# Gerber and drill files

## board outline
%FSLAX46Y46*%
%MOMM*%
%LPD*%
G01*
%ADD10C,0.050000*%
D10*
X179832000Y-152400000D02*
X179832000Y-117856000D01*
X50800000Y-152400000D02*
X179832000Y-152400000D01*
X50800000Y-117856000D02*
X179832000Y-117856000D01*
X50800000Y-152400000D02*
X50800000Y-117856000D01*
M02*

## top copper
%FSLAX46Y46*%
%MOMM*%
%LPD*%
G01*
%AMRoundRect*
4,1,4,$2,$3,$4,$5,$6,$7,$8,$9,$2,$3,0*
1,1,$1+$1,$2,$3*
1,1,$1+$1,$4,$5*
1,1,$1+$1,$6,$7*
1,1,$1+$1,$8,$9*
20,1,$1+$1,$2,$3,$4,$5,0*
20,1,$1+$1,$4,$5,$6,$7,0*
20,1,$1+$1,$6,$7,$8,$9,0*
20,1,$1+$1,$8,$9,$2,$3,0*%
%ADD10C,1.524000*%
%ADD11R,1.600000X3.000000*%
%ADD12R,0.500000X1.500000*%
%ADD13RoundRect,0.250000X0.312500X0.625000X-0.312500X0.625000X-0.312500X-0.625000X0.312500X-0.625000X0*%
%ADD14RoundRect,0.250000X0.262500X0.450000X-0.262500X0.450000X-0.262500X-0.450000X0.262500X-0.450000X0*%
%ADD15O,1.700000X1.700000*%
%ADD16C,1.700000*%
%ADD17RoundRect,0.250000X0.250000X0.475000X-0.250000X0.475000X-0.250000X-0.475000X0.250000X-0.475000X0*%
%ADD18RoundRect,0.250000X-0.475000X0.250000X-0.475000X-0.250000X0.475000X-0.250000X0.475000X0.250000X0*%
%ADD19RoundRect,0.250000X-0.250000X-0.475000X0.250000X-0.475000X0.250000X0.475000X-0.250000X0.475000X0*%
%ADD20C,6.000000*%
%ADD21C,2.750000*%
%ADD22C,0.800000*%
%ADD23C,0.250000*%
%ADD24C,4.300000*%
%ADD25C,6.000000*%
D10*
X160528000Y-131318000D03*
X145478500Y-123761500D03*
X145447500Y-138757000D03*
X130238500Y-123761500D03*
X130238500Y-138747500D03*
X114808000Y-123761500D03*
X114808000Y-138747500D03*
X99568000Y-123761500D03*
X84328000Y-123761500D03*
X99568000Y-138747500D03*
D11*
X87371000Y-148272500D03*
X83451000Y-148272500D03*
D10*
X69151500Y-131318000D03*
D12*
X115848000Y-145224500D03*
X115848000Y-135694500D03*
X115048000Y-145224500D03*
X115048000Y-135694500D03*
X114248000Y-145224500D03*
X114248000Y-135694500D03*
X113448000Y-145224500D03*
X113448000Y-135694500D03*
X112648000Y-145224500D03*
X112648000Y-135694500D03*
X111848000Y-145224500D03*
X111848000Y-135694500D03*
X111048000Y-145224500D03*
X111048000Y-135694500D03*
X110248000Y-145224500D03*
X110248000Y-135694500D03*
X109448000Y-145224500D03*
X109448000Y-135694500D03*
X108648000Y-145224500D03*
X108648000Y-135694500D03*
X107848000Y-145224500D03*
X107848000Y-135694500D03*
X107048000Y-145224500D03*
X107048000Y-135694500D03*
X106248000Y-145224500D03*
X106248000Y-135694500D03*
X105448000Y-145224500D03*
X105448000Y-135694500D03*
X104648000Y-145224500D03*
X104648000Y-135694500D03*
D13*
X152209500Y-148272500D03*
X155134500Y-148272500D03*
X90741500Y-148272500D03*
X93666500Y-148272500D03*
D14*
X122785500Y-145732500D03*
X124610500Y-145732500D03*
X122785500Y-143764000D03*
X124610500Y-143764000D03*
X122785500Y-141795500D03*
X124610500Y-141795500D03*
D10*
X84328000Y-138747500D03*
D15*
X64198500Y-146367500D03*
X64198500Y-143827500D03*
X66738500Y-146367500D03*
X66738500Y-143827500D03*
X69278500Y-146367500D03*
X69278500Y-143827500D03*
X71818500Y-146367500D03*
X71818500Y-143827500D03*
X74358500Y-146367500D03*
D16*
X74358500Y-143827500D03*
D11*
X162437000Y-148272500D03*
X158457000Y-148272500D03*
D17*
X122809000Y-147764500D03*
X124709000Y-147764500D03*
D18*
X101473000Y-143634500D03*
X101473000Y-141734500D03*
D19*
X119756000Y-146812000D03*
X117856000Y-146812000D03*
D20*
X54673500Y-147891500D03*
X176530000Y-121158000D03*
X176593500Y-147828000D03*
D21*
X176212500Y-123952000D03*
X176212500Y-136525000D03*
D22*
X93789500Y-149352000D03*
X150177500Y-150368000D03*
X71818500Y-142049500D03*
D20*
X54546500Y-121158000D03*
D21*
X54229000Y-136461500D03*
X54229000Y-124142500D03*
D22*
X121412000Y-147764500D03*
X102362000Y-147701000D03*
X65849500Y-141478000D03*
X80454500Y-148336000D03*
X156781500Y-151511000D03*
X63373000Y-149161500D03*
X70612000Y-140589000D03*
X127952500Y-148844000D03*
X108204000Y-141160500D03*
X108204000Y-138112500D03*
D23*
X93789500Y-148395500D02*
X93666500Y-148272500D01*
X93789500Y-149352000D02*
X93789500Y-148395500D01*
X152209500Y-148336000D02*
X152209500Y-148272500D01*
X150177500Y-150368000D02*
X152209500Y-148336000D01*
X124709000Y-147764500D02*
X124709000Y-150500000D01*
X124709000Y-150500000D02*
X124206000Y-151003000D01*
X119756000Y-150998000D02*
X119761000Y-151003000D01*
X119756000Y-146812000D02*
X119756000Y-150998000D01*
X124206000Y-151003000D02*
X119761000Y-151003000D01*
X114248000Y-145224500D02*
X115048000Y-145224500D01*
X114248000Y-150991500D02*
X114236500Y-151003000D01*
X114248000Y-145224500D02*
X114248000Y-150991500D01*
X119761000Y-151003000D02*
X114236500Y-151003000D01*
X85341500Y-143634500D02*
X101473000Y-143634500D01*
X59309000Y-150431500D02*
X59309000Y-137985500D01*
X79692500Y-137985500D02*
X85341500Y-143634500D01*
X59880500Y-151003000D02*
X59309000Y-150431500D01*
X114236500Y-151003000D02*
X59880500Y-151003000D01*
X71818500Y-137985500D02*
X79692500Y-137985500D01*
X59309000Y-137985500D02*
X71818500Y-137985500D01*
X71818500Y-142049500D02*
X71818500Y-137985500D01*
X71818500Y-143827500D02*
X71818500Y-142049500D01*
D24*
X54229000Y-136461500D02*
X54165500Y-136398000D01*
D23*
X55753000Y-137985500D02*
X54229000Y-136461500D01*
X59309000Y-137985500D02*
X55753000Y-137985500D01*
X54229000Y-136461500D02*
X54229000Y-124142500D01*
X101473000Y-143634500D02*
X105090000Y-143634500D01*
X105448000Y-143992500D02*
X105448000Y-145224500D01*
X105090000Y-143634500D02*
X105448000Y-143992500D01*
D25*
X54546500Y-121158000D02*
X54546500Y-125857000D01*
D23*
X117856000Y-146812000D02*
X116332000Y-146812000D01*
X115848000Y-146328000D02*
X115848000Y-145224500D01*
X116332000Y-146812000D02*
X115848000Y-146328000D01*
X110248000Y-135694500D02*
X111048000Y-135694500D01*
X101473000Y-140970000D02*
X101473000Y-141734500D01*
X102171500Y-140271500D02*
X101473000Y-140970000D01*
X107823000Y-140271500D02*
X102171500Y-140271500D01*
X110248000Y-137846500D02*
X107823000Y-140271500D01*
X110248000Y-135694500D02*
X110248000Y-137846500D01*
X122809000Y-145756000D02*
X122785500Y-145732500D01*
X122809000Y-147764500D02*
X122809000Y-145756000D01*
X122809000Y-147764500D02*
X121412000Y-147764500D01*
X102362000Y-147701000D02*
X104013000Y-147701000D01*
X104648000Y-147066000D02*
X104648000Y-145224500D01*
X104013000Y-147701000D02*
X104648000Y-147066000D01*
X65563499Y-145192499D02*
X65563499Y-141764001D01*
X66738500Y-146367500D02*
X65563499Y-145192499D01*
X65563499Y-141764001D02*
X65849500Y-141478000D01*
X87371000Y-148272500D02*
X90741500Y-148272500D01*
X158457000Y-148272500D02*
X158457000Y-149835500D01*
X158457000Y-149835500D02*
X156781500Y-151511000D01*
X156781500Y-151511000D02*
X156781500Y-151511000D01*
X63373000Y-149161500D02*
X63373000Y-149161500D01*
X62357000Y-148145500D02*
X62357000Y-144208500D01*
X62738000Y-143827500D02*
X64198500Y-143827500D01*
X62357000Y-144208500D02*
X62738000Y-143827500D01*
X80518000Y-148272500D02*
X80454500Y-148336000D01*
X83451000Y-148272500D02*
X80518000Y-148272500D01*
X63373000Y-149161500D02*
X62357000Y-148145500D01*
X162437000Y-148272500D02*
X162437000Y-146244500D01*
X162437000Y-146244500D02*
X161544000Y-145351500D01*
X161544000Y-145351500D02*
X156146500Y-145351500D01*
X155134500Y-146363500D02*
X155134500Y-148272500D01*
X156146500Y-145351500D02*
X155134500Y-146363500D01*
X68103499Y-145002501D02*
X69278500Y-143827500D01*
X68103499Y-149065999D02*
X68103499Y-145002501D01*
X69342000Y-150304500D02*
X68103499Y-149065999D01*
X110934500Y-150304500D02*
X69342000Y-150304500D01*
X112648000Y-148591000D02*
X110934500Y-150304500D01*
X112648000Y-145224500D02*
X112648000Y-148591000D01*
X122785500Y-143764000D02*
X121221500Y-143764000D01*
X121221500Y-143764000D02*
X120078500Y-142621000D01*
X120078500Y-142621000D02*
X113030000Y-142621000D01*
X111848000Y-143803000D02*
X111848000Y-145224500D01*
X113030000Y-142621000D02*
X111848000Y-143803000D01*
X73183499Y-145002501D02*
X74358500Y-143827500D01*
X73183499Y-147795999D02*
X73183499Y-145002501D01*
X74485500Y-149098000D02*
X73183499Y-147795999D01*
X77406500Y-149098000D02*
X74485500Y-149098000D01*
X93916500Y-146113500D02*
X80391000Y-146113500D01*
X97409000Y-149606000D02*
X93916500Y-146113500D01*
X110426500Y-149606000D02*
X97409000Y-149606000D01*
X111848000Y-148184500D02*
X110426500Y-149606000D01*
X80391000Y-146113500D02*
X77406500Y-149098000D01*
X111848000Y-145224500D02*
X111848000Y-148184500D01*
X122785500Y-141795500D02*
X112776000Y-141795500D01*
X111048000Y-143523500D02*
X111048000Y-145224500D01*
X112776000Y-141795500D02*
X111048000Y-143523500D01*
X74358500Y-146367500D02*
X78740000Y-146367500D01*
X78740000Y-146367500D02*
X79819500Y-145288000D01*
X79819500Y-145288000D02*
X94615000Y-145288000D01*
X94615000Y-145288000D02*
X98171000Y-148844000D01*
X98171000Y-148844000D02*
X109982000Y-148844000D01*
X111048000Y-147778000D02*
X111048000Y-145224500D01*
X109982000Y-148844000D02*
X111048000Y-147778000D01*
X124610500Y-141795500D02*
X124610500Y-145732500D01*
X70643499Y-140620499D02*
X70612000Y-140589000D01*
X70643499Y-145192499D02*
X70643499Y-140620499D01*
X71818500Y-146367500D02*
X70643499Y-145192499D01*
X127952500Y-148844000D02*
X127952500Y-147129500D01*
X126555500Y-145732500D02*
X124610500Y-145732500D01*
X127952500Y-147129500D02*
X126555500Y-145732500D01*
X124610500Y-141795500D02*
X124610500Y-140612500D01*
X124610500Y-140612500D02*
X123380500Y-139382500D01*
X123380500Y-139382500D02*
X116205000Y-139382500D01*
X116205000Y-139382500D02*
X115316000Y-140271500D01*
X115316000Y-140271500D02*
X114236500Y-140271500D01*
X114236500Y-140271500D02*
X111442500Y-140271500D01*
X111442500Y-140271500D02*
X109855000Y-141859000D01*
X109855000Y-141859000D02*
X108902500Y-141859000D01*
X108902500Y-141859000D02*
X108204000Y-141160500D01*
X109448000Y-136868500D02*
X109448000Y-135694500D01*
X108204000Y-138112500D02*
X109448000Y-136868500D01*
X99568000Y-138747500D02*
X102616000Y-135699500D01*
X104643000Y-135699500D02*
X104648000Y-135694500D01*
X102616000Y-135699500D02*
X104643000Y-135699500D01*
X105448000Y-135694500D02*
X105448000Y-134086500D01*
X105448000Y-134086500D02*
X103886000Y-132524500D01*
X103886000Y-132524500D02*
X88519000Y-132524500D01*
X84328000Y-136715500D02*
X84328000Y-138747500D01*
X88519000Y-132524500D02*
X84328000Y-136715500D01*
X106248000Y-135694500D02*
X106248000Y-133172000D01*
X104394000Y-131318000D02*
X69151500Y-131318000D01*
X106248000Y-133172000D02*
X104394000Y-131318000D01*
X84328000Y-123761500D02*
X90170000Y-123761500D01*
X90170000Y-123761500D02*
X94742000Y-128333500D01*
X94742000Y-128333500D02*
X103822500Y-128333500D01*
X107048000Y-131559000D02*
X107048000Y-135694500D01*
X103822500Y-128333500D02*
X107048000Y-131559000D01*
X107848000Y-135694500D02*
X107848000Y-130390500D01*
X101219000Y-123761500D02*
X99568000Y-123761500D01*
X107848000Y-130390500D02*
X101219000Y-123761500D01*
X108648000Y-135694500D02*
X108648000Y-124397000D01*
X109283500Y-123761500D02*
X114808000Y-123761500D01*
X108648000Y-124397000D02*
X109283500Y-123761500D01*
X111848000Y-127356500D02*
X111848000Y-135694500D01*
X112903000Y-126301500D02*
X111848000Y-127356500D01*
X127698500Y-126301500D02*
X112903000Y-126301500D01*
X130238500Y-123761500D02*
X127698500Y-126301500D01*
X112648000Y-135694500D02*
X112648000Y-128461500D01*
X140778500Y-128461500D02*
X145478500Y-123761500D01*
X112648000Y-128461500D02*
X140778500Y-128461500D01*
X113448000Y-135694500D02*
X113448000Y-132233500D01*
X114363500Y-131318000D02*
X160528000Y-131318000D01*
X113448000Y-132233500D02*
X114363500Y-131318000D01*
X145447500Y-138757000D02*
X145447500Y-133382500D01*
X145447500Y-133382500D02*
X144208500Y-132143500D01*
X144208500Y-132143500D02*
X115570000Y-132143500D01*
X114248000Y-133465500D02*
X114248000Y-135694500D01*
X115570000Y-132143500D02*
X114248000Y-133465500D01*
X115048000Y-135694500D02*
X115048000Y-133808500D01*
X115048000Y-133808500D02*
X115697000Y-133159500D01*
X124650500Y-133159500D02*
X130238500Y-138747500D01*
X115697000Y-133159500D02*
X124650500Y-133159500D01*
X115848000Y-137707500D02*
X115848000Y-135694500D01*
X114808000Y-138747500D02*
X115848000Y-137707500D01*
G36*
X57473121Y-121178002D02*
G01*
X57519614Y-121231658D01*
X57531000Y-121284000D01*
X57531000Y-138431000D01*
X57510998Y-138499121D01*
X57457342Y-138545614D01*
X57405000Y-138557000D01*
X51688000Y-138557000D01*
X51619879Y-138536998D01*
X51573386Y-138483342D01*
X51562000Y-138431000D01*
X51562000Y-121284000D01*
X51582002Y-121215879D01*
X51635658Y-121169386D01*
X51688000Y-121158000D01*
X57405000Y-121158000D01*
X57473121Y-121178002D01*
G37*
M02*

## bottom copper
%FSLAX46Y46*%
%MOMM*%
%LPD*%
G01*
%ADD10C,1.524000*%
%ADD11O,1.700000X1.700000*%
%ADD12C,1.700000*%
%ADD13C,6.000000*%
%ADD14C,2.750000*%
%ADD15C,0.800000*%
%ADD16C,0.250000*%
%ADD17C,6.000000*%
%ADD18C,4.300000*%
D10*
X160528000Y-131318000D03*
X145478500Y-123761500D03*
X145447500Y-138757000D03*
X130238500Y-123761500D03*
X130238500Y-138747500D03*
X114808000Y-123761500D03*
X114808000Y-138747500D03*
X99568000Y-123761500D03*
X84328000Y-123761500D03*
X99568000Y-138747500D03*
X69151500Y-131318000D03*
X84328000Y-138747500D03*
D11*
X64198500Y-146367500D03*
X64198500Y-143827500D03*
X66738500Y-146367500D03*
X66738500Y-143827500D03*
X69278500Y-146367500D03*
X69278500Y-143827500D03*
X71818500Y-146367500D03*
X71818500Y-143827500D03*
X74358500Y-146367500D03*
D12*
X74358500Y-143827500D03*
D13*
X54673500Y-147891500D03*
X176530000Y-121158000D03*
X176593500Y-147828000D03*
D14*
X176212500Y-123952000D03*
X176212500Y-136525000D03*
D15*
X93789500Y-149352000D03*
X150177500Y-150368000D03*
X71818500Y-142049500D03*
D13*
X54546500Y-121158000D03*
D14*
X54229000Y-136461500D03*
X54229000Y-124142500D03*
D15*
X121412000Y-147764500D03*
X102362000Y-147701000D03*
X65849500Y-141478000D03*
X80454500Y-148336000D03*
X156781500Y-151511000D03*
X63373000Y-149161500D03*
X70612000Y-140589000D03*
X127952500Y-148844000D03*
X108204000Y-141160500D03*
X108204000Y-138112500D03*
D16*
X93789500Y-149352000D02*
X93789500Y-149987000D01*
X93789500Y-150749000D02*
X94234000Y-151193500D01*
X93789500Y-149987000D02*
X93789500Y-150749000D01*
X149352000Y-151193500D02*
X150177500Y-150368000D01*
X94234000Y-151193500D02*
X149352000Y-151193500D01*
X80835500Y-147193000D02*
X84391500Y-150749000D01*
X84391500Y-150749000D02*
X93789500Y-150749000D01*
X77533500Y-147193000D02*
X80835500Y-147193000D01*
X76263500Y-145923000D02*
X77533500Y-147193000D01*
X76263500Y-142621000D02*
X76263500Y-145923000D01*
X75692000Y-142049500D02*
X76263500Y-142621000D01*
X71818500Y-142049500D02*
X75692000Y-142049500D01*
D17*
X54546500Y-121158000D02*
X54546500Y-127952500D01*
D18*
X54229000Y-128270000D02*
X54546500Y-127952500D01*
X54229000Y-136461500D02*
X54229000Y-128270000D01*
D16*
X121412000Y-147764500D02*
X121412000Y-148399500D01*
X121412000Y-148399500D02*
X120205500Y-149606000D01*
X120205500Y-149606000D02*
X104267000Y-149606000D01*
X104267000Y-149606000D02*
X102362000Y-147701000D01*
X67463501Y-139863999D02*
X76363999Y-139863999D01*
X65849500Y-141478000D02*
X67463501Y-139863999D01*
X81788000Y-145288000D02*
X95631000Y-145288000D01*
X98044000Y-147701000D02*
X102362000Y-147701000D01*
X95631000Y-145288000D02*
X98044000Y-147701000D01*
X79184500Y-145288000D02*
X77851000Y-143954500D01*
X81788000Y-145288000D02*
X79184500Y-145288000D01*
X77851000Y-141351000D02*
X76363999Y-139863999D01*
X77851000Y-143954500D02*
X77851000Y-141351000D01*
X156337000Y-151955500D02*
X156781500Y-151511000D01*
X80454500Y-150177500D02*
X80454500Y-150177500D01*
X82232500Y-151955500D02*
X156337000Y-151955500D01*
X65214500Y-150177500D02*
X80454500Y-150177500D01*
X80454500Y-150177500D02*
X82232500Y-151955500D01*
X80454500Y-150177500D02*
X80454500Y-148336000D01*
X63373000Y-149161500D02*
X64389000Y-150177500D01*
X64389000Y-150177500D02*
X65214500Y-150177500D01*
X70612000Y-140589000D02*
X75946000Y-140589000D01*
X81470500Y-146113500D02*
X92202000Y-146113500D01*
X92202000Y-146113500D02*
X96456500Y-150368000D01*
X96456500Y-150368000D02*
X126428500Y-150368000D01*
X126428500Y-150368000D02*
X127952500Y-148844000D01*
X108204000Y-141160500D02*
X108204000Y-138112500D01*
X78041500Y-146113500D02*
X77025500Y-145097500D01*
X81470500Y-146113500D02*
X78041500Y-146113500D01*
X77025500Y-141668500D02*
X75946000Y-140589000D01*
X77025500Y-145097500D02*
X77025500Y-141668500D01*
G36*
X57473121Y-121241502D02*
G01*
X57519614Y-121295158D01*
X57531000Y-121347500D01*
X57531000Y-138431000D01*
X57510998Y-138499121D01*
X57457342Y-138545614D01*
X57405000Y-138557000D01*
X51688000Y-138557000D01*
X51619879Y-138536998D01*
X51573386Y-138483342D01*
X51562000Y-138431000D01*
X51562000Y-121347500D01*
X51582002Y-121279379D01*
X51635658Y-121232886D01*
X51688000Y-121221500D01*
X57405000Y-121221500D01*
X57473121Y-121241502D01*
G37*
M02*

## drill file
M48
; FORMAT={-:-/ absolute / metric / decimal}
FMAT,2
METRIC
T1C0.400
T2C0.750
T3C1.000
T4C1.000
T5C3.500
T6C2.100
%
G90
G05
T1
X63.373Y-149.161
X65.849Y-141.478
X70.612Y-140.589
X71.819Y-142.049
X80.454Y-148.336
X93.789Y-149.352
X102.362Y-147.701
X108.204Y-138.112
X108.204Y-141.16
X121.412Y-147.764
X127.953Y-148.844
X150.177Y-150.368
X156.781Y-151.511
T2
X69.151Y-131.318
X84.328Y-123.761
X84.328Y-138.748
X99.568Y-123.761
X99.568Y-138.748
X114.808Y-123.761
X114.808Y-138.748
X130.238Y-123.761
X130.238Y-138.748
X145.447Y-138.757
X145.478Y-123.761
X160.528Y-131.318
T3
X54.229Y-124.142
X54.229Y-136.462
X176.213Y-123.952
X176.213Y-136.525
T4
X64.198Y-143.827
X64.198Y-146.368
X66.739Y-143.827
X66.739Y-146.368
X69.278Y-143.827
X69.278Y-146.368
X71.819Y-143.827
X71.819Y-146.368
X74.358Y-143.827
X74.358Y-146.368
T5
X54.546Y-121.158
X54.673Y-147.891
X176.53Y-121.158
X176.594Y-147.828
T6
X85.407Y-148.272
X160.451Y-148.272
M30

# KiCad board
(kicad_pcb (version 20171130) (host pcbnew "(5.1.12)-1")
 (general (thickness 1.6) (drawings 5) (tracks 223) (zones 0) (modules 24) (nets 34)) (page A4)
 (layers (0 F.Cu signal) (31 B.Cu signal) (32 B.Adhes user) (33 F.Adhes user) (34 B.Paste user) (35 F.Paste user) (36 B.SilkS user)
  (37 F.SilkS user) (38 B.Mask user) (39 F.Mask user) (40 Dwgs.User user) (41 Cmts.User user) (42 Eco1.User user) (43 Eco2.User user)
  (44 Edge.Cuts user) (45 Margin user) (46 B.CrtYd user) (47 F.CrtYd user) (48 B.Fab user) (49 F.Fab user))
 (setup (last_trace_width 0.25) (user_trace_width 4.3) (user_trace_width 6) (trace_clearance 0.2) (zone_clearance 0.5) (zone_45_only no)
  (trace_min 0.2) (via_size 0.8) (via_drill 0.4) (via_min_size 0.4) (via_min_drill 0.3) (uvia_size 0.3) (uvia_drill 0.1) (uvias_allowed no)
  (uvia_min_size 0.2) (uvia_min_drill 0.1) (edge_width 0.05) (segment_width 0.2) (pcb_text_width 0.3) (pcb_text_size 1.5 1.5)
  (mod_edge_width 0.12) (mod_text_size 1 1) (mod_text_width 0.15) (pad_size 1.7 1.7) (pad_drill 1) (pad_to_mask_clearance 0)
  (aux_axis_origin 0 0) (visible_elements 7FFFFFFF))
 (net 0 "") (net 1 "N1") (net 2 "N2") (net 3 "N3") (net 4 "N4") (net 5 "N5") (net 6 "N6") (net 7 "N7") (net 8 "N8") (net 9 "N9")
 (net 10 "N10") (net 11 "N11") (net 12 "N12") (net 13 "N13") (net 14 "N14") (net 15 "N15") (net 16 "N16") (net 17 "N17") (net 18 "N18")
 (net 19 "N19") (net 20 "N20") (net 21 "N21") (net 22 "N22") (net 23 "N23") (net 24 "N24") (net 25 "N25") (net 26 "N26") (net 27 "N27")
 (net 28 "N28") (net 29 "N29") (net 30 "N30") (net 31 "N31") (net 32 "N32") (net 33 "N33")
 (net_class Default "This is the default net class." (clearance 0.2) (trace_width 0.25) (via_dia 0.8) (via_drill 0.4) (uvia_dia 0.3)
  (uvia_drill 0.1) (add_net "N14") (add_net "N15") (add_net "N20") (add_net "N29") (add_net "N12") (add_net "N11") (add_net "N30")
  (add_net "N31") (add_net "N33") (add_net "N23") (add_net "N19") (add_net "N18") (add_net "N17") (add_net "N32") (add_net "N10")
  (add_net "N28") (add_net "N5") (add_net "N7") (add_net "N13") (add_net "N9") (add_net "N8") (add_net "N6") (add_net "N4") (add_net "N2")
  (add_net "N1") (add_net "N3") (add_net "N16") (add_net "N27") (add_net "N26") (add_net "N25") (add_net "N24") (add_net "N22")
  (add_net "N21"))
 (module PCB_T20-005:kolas (layer B.Cu) (at 160.528 131.318 270)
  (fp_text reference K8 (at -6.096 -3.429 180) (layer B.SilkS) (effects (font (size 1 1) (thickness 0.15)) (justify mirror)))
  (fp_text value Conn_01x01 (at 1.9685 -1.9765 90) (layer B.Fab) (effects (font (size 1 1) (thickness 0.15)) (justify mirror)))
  (pad 1 thru_hole circle (at 0 0 270) (size 1.524 1.524) (drill 0.75) (layers *.Cu *.Mask) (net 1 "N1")))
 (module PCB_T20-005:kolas (layer B.Cu) (at 145.4785 123.7615)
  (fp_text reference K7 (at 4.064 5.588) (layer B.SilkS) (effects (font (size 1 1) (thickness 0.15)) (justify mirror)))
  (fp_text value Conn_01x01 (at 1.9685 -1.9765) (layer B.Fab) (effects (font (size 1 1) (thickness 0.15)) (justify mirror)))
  (pad 1 thru_hole circle (at 0 0) (size 1.524 1.524) (drill 0.75) (layers *.Cu *.Mask) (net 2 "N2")))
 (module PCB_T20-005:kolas (layer B.Cu) (at 145.4475 138.757)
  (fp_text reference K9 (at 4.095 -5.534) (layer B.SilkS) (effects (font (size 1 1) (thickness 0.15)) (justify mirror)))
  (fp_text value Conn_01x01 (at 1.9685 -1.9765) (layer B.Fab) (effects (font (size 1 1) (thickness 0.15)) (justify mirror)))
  (pad 1 thru_hole circle (at 0 0) (size 1.524 1.524) (drill 0.75) (layers *.Cu *.Mask) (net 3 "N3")))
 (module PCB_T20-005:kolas (layer B.Cu) (at 130.2385 123.7615)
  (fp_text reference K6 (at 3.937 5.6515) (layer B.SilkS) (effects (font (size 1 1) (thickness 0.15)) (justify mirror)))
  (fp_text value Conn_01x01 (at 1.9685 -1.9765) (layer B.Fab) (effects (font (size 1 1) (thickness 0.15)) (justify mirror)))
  (pad 1 thru_hole circle (at 0 0) (size 1.524 1.524) (drill 0.75) (layers *.Cu *.Mask) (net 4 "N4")))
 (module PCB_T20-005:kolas (layer B.Cu) (at 130.2385 138.7475)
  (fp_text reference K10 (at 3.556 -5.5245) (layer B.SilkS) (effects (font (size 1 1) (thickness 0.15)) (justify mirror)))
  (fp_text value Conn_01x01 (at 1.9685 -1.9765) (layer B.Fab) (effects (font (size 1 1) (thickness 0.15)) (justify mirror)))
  (pad 1 thru_hole circle (at 0 0) (size 1.524 1.524) (drill 0.75) (layers *.Cu *.Mask) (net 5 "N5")))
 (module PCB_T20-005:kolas (layer B.Cu) (at 114.808 123.7615)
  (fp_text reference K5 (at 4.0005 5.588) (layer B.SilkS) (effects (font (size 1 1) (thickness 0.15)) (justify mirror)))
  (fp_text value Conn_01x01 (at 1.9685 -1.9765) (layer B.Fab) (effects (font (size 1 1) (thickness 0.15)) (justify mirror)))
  (pad 1 thru_hole circle (at 0 0) (size 1.524 1.524) (drill 0.75) (layers *.Cu *.Mask) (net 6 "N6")))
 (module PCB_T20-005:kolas (layer B.Cu) (at 114.808 138.7475)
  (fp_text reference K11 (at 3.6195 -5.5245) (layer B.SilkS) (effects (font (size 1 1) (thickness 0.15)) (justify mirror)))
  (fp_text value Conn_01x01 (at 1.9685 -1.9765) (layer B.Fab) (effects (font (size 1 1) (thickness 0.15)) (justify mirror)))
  (pad 1 thru_hole circle (at 0 0) (size 1.524 1.524) (drill 0.75) (layers *.Cu *.Mask) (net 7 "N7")))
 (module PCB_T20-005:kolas (layer B.Cu) (at 99.568 123.7615)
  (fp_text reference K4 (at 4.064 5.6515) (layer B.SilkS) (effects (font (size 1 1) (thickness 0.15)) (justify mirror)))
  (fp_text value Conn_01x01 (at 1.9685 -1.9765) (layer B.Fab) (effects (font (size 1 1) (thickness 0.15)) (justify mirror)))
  (pad 1 thru_hole circle (at 0 0) (size 1.524 1.524) (drill 0.75) (layers *.Cu *.Mask) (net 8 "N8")))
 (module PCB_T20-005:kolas (layer B.Cu) (at 84.328 123.7615)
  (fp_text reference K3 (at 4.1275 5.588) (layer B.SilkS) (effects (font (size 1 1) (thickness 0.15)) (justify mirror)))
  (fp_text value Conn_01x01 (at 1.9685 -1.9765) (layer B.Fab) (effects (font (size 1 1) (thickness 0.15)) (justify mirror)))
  (pad 1 thru_hole circle (at 0 0) (size 1.524 1.524) (drill 0.75) (layers *.Cu *.Mask) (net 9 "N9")))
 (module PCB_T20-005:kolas (layer B.Cu) (at 99.568 138.7475)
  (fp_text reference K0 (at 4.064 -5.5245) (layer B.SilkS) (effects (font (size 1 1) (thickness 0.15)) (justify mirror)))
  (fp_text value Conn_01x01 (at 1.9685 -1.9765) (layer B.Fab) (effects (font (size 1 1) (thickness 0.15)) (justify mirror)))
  (pad 1 thru_hole circle (at 0 0) (size 1.524 1.524) (drill 0.75) (layers *.Cu *.Mask) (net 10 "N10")))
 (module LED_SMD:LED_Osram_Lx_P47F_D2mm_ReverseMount (layer F.Cu) (at 85.4075 148.2725)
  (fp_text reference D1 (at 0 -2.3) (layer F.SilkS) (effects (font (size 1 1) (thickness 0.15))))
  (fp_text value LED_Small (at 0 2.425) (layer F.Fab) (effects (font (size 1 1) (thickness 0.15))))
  (pad 2 smd rect (at 1.9635 0) (size 1.6 3) (layers F.Cu) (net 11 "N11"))
  (pad 1 smd rect (at -1.9565 0) (size 1.6 3) (layers F.Cu) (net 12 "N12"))
  (pad "" np_thru_hole circle (at 0 0) (size 2.1 2.1) (drill 2.1) (layers *.Cu *.Mask))
  (pad "" smd rect (at -1.9565 0) (size 1.6 3) (layers F.Paste F.Mask))
  (pad "" smd rect (at 1.9635 0) (size 1.6 3) (layers F.Paste F.Mask)))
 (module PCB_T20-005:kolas (layer B.Cu) (at 69.1515 131.318 90)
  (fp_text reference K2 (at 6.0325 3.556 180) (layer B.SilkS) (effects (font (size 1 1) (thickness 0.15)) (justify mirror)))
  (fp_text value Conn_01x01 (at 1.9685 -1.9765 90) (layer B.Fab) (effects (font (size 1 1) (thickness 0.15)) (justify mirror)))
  (pad 1 thru_hole circle (at 0 0 90) (size 1.524 1.524) (drill 0.75) (layers *.Cu *.Mask) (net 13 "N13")))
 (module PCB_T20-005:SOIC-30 (layer F.Cu) (at 110.248 140.4595)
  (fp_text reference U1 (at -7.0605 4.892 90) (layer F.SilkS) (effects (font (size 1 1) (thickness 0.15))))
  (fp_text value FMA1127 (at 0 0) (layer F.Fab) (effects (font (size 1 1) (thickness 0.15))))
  (pad 15 smd rect (at 5.6 4.765) (size 0.5 1.5) (layers F.Cu F.Paste F.Mask) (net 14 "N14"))
  (pad 16 smd rect (at 5.6 -4.765) (size 0.5 1.5) (layers F.Cu F.Paste F.Mask) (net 7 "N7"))
  (pad 14 smd rect (at 4.8 4.765) (size 0.5 1.5) (layers F.Cu F.Paste F.Mask) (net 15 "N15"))
  (pad 17 smd rect (at 4.8 -4.765) (size 0.5 1.5) (layers F.Cu F.Paste F.Mask) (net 5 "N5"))
  (pad 13 smd rect (at 4 4.765) (size 0.5 1.5) (layers F.Cu F.Paste F.Mask) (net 15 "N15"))
  (pad 18 smd rect (at 4 -4.765) (size 0.5 1.5) (layers F.Cu F.Paste F.Mask) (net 3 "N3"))
  (pad 12 smd rect (at 3.2 4.765) (size 0.5 1.5) (layers F.Cu F.Paste F.Mask) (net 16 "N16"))
  (pad 19 smd rect (at 3.2 -4.765) (size 0.5 1.5) (layers F.Cu F.Paste F.Mask) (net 1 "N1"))
  (pad 11 smd rect (at 2.4 4.765) (size 0.5 1.5) (layers F.Cu F.Paste F.Mask) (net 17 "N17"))
  (pad 20 smd rect (at 2.4 -4.765) (size 0.5 1.5) (layers F.Cu F.Paste F.Mask) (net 2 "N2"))
  (pad 10 smd rect (at 1.6 4.765) (size 0.5 1.5) (layers F.Cu F.Paste F.Mask) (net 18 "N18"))
  (pad 21 smd rect (at 1.6 -4.765) (size 0.5 1.5) (layers F.Cu F.Paste F.Mask) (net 4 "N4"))
  (pad 9 smd rect (at 0.8 4.765) (size 0.5 1.5) (layers F.Cu F.Paste F.Mask) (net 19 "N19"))
  (pad 22 smd rect (at 0.8 -4.765) (size 0.5 1.5) (layers F.Cu F.Paste F.Mask) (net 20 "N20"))
  (pad 8 smd rect (at 0 4.765) (size 0.5 1.5) (layers F.Cu F.Paste F.Mask) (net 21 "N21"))
  (pad 23 smd rect (at 0 -4.765) (size 0.5 1.5) (layers F.Cu F.Paste F.Mask) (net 20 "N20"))
  (pad 7 smd rect (at -0.8 4.765) (size 0.5 1.5) (layers F.Cu F.Paste F.Mask) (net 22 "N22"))
  (pad 24 smd rect (at -0.8 -4.765) (size 0.5 1.5) (layers F.Cu F.Paste F.Mask) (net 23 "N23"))
  (pad 6 smd rect (at -1.6 4.765) (size 0.5 1.5) (layers F.Cu F.Paste F.Mask) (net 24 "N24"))
  (pad 25 smd rect (at -1.6 -4.765) (size 0.5 1.5) (layers F.Cu F.Paste F.Mask) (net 6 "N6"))
  (pad 5 smd rect (at -2.4 4.765) (size 0.5 1.5) (layers F.Cu F.Paste F.Mask) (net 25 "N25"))
  (pad 26 smd rect (at -2.4 -4.765) (size 0.5 1.5) (layers F.Cu F.Paste F.Mask) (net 8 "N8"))
  (pad 4 smd rect (at -3.2 4.765) (size 0.5 1.5) (layers F.Cu F.Paste F.Mask) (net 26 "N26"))
  (pad 27 smd rect (at -3.2 -4.765) (size 0.5 1.5) (layers F.Cu F.Paste F.Mask) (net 9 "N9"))
  (pad 3 smd rect (at -4 4.765) (size 0.5 1.5) (layers F.Cu F.Paste F.Mask) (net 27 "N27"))
  (pad 28 smd rect (at -4 -4.765) (size 0.5 1.5) (layers F.Cu F.Paste F.Mask) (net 13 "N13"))
  (pad 2 smd rect (at -4.8 4.765) (size 0.5 1.5) (layers F.Cu F.Paste F.Mask) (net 15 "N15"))
  (pad 29 smd rect (at -4.8 -4.765) (size 0.5 1.5) (layers F.Cu F.Paste F.Mask) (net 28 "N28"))
  (pad 1 smd rect (at -5.6 4.765) (size 0.5 1.5) (layers F.Cu F.Paste F.Mask) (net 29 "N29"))
  (pad 30 smd rect (at -5.6 -4.765) (size 0.5 1.5) (layers F.Cu F.Paste F.Mask) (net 10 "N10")))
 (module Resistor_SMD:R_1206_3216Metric (layer F.Cu) (at 153.672 148.2725 180)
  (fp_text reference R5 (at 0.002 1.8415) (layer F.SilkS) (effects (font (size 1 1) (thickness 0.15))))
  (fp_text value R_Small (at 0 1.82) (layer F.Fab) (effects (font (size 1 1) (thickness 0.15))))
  (pad 2 smd roundrect (at 1.4625 0 180) (size 1.125 1.75) (layers F.Cu F.Paste F.Mask) (roundrect_rratio 0.222222) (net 15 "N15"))
  (pad 1 smd roundrect (at -1.4625 0 180) (size 1.125 1.75) (layers F.Cu F.Paste F.Mask) (roundrect_rratio 0.222222) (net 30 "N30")))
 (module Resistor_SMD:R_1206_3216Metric (layer F.Cu) (at 92.204 148.2725 180)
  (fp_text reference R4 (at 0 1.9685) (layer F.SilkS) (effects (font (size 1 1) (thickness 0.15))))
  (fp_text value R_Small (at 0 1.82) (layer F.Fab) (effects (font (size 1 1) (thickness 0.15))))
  (pad 2 smd roundrect (at 1.4625 0 180) (size 1.125 1.75) (layers F.Cu F.Paste F.Mask) (roundrect_rratio 0.222222) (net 11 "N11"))
  (pad 1 smd roundrect (at -1.4625 0 180) (size 1.125 1.75) (layers F.Cu F.Paste F.Mask) (roundrect_rratio 0.222222) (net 15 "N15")))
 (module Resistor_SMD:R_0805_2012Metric (layer F.Cu) (at 123.698 145.7325 180)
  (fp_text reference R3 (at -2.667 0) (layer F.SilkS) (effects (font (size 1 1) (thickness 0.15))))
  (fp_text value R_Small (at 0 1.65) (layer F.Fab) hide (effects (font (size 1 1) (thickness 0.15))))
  (pad 2 smd roundrect (at 0.9125 0 180) (size 1.025 1.4) (layers F.Cu F.Paste F.Mask) (roundrect_rratio 0.243902) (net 29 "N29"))
  (pad 1 smd roundrect (at -0.9125 0 180) (size 1.025 1.4) (layers F.Cu F.Paste F.Mask) (roundrect_rratio 0.243902) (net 23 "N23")))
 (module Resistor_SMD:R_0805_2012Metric (layer F.Cu) (at 123.698 143.764 180)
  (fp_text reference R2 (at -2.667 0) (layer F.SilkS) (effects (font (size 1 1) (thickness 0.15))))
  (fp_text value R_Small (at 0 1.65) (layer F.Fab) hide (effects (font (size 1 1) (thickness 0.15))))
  (pad 2 smd roundrect (at 0.9125 0 180) (size 1.025 1.4) (layers F.Cu F.Paste F.Mask) (roundrect_rratio 0.243902) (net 18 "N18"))
  (pad 1 smd roundrect (at -0.9125 0 180) (size 1.025 1.4) (layers F.Cu F.Paste F.Mask) (roundrect_rratio 0.243902) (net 23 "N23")))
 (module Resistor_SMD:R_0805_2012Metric (layer F.Cu) (at 123.698 141.7955 180)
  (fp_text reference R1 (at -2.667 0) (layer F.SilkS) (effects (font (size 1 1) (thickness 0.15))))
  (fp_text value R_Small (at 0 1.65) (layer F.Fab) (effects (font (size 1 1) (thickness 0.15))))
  (pad 2 smd roundrect (at 0.9125 0 180) (size 1.025 1.4) (layers F.Cu F.Paste F.Mask) (roundrect_rratio 0.243902) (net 19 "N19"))
  (pad 1 smd roundrect (at -0.9125 0 180) (size 1.025 1.4) (layers F.Cu F.Paste F.Mask) (roundrect_rratio 0.243902) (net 23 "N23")))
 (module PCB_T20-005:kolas (layer B.Cu) (at 84.328 138.7475)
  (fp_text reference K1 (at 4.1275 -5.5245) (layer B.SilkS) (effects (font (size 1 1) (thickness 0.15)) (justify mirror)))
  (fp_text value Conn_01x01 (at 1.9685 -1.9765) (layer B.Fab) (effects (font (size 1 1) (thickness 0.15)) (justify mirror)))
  (pad 1 thru_hole circle (at 0 0) (size 1.524 1.524) (drill 0.75) (layers *.Cu *.Mask) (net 28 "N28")))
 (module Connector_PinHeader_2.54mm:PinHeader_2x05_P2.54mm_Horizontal (layer F.Cu) (at 74.3585 143.8275 270)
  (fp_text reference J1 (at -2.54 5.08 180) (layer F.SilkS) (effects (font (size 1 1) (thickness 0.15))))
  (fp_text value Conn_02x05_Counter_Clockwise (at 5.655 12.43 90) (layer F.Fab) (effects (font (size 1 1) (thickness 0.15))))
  (pad 1 thru_hole oval (at 2.54 10.16 270) (size 1.7 1.7) (drill 1) (layers *.Cu *.Mask) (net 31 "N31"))
  (pad 10 thru_hole oval (at 0 10.16 270) (size 1.7 1.7) (drill 1) (layers *.Cu *.Mask) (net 12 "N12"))
  (pad 2 thru_hole oval (at 2.54 7.62 270) (size 1.7 1.7) (drill 1) (layers *.Cu *.Mask) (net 29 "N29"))
  (pad 9 thru_hole oval (at 0 7.62 270) (size 1.7 1.7) (drill 1) (layers *.Cu *.Mask) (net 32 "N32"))
  (pad 3 thru_hole oval (at 2.54 5.08 270) (size 1.7 1.7) (drill 1) (layers *.Cu *.Mask) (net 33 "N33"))
  (pad 8 thru_hole oval (at 0 5.08 270) (size 1.7 1.7) (drill 1) (layers *.Cu *.Mask) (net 17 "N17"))
  (pad 4 thru_hole oval (at 2.54 2.54 270) (size 1.7 1.7) (drill 1) (layers *.Cu *.Mask) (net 23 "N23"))
  (pad 7 thru_hole oval (at 0 2.54 270) (size 1.7 1.7) (drill 1) (layers *.Cu *.Mask) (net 15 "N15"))
  (pad 5 thru_hole oval (at 2.54 0 270) (size 1.7 1.7) (drill 1) (layers *.Cu *.Mask) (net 19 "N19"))
  (pad 6 thru_hole circle (at 0 0 270) (size 1.7 1.7) (drill 1) (layers *.Cu *.Mask) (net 18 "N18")))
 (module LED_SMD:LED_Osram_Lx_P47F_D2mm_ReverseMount (layer F.Cu) (at 160.4505 148.2725)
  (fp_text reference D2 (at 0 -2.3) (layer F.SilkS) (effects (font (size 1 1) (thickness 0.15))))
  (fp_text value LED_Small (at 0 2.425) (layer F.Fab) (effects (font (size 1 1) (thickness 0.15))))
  (pad 2 smd rect (at 1.9865 0) (size 1.6 3) (layers F.Cu) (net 30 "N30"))
  (pad 1 smd rect (at -1.9935 0) (size 1.6 3) (layers F.Cu) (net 12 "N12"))
  (pad "" np_thru_hole circle (at 0 0) (size 2.1 2.1) (drill 2.1) (layers *.Cu *.Mask))
  (pad "" smd rect (at -1.9935 0) (size 1.6 3) (layers F.Paste F.Mask))
  (pad "" smd rect (at 1.9865 0) (size 1.6 3) (layers F.Paste F.Mask)))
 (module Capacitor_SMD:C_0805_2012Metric (layer F.Cu) (at 123.759 147.7645 180)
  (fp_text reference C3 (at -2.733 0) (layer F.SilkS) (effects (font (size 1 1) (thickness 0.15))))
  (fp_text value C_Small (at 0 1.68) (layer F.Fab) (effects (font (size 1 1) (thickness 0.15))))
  (pad 2 smd roundrect (at 0.95 0 180) (size 1 1.45) (layers F.Cu F.Paste F.Mask) (roundrect_rratio 0.25) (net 29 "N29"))
  (pad 1 smd roundrect (at -0.95 0 180) (size 1 1.45) (layers F.Cu F.Paste F.Mask) (roundrect_rratio 0.25) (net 15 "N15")))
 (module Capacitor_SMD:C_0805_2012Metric (layer F.Cu) (at 101.473 142.6845 270)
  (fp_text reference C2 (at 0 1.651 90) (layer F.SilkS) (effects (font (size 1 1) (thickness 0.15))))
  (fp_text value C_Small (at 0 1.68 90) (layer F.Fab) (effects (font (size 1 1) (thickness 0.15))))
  (pad 2 smd roundrect (at 0.95 0 270) (size 1 1.45) (layers F.Cu F.Paste F.Mask) (roundrect_rratio 0.25) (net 15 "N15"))
  (pad 1 smd roundrect (at -0.95 0 270) (size 1 1.45) (layers F.Cu F.Paste F.Mask) (roundrect_rratio 0.25) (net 20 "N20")))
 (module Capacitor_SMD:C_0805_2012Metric (layer F.Cu) (at 118.806 146.812)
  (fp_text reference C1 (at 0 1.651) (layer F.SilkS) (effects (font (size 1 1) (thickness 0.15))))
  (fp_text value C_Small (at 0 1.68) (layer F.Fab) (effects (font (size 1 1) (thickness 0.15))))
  (pad 2 smd roundrect (at 0.95 0) (size 1 1.45) (layers F.Cu F.Paste F.Mask) (roundrect_rratio 0.25) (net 15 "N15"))
  (pad 1 smd roundrect (at -0.95 0) (size 1 1.45) (layers F.Cu F.Paste F.Mask) (roundrect_rratio 0.25) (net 14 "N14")))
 (gr_line (start 179.832 152.4) (end 179.832 117.856) (layer Edge.Cuts) (width 0.05))
 (gr_line (start 50.8 152.4) (end 179.832 152.4) (layer Edge.Cuts) (width 0.05))
 (gr_line (start 50.8 117.856) (end 179.832 117.856) (layer Edge.Cuts) (width 0.05))
 (gr_line (start 50.8 152.4) (end 50.8 117.856) (layer Edge.Cuts) (width 0.05))
 (via (at 54.6735 147.8915) (size 6) (drill 3.5) (layers F.Cu B.Cu) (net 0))
 (via (at 176.53 121.158) (size 6) (drill 3.5) (layers F.Cu B.Cu) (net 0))
 (via (at 176.5935 147.828) (size 6) (drill 3.5) (layers F.Cu B.Cu) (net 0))
 (via (at 176.2125 123.952) (size 2.75) (drill 1) (layers F.Cu B.Cu) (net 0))
 (via (at 176.2125 136.525) (size 2.75) (drill 1) (layers F.Cu B.Cu) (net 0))
 (via (at 93.7895 149.352) (size 0.8) (drill 0.4) (layers F.Cu B.Cu) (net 15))
 (segment (start 93.7895 148.3955) (end 93.6665 148.2725) (width 0.25) (layer F.Cu) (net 15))
 (segment (start 93.7895 149.352) (end 93.7895 148.3955) (width 0.25) (layer F.Cu) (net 15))
 (segment (start 93.7895 149.352) (end 93.7895 149.987) (width 0.25) (layer B.Cu) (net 15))
 (segment (start 93.7895 150.749) (end 94.234 151.1935) (width 0.25) (layer B.Cu) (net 15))
 (segment (start 93.7895 149.987) (end 93.7895 150.749) (width 0.25) (layer B.Cu) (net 15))
 (via (at 150.1775 150.368) (size 0.8) (drill 0.4) (layers F.Cu B.Cu) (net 15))
 (segment (start 149.352 151.1935) (end 150.1775 150.368) (width 0.25) (layer B.Cu) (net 15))
 (segment (start 94.234 151.1935) (end 149.352 151.1935) (width 0.25) (layer B.Cu) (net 15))
 (segment (start 152.2095 148.336) (end 152.2095 148.2725) (width 0.25) (layer F.Cu) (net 15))
 (segment (start 150.1775 150.368) (end 152.2095 148.336) (width 0.25) (layer F.Cu) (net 15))
 (segment (start 124.709 147.7645) (end 124.709 150.5) (width 0.25) (layer F.Cu) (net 15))
 (segment (start 124.709 150.5) (end 124.206 151.003) (width 0.25) (layer F.Cu) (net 15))
 (segment (start 119.756 150.998) (end 119.761 151.003) (width 0.25) (layer F.Cu) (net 15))
 (segment (start 119.756 146.812) (end 119.756 150.998) (width 0.25) (layer F.Cu) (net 15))
 (segment (start 124.206 151.003) (end 119.761 151.003) (width 0.25) (layer F.Cu) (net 15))
 (segment (start 114.248 145.2245) (end 115.048 145.2245) (width 0.25) (layer F.Cu) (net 15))
 (segment (start 114.248 150.9915) (end 114.2365 151.003) (width 0.25) (layer F.Cu) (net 15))
 (segment (start 114.248 145.2245) (end 114.248 150.9915) (width 0.25) (layer F.Cu) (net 15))
 (segment (start 119.761 151.003) (end 114.2365 151.003) (width 0.25) (layer F.Cu) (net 15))
 (segment (start 85.3415 143.6345) (end 101.473 143.6345) (width 0.25) (layer F.Cu) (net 15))
 (segment (start 59.309 150.4315) (end 59.309 137.9855) (width 0.25) (layer F.Cu) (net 15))
 (segment (start 79.6925 137.9855) (end 85.3415 143.6345) (width 0.25) (layer F.Cu) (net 15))
 (segment (start 59.8805 151.003) (end 59.309 150.4315) (width 0.25) (layer F.Cu) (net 15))
 (segment (start 114.2365 151.003) (end 59.8805 151.003) (width 0.25) (layer F.Cu) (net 15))
 (segment (start 71.8185 137.9855) (end 79.6925 137.9855) (width 0.25) (layer F.Cu) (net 15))
 (segment (start 59.309 137.9855) (end 71.8185 137.9855) (width 0.25) (layer F.Cu) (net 15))
 (via (at 71.8185 142.0495) (size 0.8) (drill 0.4) (layers F.Cu B.Cu) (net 15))
 (segment (start 71.8185 142.0495) (end 71.8185 137.9855) (width 0.25) (layer F.Cu) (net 15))
 (segment (start 71.8185 143.8275) (end 71.8185 142.0495) (width 0.25) (layer F.Cu) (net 15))
 (via (at 54.5465 121.158) (size 6) (drill 3.5) (layers F.Cu B.Cu) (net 15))
 (via (at 54.229 136.4615) (size 2.75) (drill 1) (layers F.Cu B.Cu) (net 15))
 (via (at 54.229 124.1425) (size 2.75) (drill 1) (layers F.Cu B.Cu) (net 15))
 (segment (start 54.229 136.4615) (end 54.1655 136.398) (width 4.3) (layer F.Cu) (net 15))
 (segment (start 55.753 137.9855) (end 54.229 136.4615) (width 0.25) (layer F.Cu) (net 15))
 (segment (start 59.309 137.9855) (end 55.753 137.9855) (width 0.25) (layer F.Cu) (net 15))
 (segment (start 54.229 136.4615) (end 54.229 124.1425) (width 0.25) (layer F.Cu) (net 15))
 (segment (start 101.473 143.6345) (end 105.09 143.6345) (width 0.25) (layer F.Cu) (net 15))
 (segment (start 105.448 143.9925) (end 105.448 145.2245) (width 0.25) (layer F.Cu) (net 15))
 (segment (start 105.09 143.6345) (end 105.448 143.9925) (width 0.25) (layer F.Cu) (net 15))
 (segment (start 80.8355 147.193) (end 84.3915 150.749) (width 0.25) (layer B.Cu) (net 15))
 (segment (start 84.3915 150.749) (end 93.7895 150.749) (width 0.25) (layer B.Cu) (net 15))
 (segment (start 77.5335 147.193) (end 80.8355 147.193) (width 0.25) (layer B.Cu) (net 15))
 (segment (start 76.2635 145.923) (end 77.5335 147.193) (width 0.25) (layer B.Cu) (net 15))
 (segment (start 76.2635 142.621) (end 76.2635 145.923) (width 0.25) (layer B.Cu) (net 15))
 (segment (start 75.692 142.0495) (end 76.2635 142.621) (width 0.25) (layer B.Cu) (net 15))
 (segment (start 71.8185 142.0495) (end 75.692 142.0495) (width 0.25) (layer B.Cu) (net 15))
 (segment (start 54.5465 121.158) (end 54.5465 125.857) (width 6) (layer F.Cu) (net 15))
 (segment (start 54.5465 121.158) (end 54.5465 127.9525) (width 6) (layer B.Cu) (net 15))
 (segment (start 54.229 128.27) (end 54.5465 127.9525) (width 4.3) (layer B.Cu) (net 15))
 (segment (start 54.229 136.4615) (end 54.229 128.27) (width 4.3) (layer B.Cu) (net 15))
 (segment (start 117.856 146.812) (end 116.332 146.812) (width 0.25) (layer F.Cu) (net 14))
 (segment (start 115.848 146.328) (end 115.848 145.2245) (width 0.25) (layer F.Cu) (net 14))
 (segment (start 116.332 146.812) (end 115.848 146.328) (width 0.25) (layer F.Cu) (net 14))
 (segment (start 110.248 135.6945) (end 111.048 135.6945) (width 0.25) (layer F.Cu) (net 20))
 (segment (start 101.473 140.97) (end 101.473 141.7345) (width 0.25) (layer F.Cu) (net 20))
 (segment (start 102.1715 140.2715) (end 101.473 140.97) (width 0.25) (layer F.Cu) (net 20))
 (segment (start 107.823 140.2715) (end 102.1715 140.2715) (width 0.25) (layer F.Cu) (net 20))
 (segment (start 110.248 137.8465) (end 107.823 140.2715) (width 0.25) (layer F.Cu) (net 20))
 (segment (start 110.248 135.6945) (end 110.248 137.8465) (width 0.25) (layer F.Cu) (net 20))
 (segment (start 122.809 145.756) (end 122.7855 145.7325) (width 0.25) (layer F.Cu) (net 29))
 (segment (start 122.809 147.7645) (end 122.809 145.756) (width 0.25) (layer F.Cu) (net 29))
 (via (at 121.412 147.7645) (size 0.8) (drill 0.4) (layers F.Cu B.Cu) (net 29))
 (segment (start 122.809 147.7645) (end 121.412 147.7645) (width 0.25) (layer F.Cu) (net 29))
 (segment (start 121.412 147.7645) (end 121.412 148.3995) (width 0.25) (layer B.Cu) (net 29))
 (segment (start 121.412 148.3995) (end 120.2055 149.606) (width 0.25) (layer B.Cu) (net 29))
 (segment (start 120.2055 149.606) (end 104.267 149.606) (width 0.25) (layer B.Cu) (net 29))
 (via (at 102.362 147.701) (size 0.8) (drill 0.4) (layers F.Cu B.Cu) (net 29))
 (segment (start 104.267 149.606) (end 102.362 147.701) (width 0.25) (layer B.Cu) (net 29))
 (segment (start 102.362 147.701) (end 104.013 147.701) (width 0.25) (layer F.Cu) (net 29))
 (segment (start 104.648 147.066) (end 104.648 145.2245) (width 0.25) (layer F.Cu) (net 29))
 (segment (start 104.013 147.701) (end 104.648 147.066) (width 0.25) (layer F.Cu) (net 29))
 (segment (start 65.563499 145.192499) (end 65.563499 141.764001) (width 0.25) (layer F.Cu) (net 29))
 (segment (start 66.7385 146.3675) (end 65.563499 145.192499) (width 0.25) (layer F.Cu) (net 29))
 (via (at 65.8495 141.478) (size 0.8) (drill 0.4) (layers F.Cu B.Cu) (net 29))
 (segment (start 65.563499 141.764001) (end 65.8495 141.478) (width 0.25) (layer F.Cu) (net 29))
 (segment (start 67.463501 139.863999) (end 76.363999 139.863999) (width 0.25) (layer B.Cu) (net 29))
 (segment (start 65.8495 141.478) (end 67.463501 139.863999) (width 0.25) (layer B.Cu) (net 29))
 (segment (start 81.788 145.288) (end 95.631 145.288) (width 0.25) (layer B.Cu) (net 29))
 (segment (start 98.044 147.701) (end 102.362 147.701) (width 0.25) (layer B.Cu) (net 29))
 (segment (start 95.631 145.288) (end 98.044 147.701) (width 0.25) (layer B.Cu) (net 29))
 (segment (start 79.1845 145.288) (end 77.851 143.9545) (width 0.25) (layer B.Cu) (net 29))
 (segment (start 81.788 145.288) (end 79.1845 145.288) (width 0.25) (layer B.Cu) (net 29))
 (segment (start 77.851 141.351) (end 76.363999 139.863999) (width 0.25) (layer B.Cu) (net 29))
 (segment (start 77.851 143.9545) (end 77.851 141.351) (width 0.25) (layer B.Cu) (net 29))
 (segment (start 87.371 148.2725) (end 90.7415 148.2725) (width 0.25) (layer F.Cu) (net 11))
 (via (at 80.4545 148.336) (size 0.8) (drill 0.4) (layers F.Cu B.Cu) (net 12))
 (segment (start 158.457 148.2725) (end 158.457 149.8355) (width 0.25) (layer F.Cu) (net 12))
 (segment (start 158.457 149.8355) (end 156.7815 151.511) (width 0.25) (layer F.Cu) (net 12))
 (segment (start 156.7815 151.511) (end 156.7815 151.511) (width 0.25) (layer F.Cu) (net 12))
 (via (at 156.7815 151.511) (size 0.8) (drill 0.4) (layers F.Cu B.Cu) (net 12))
 (segment (start 156.337 151.9555) (end 156.7815 151.511) (width 0.25) (layer B.Cu) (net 12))
 (segment (start 80.4545 150.1775) (end 80.4545 150.1775) (width 0.25) (layer B.Cu) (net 12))
 (segment (start 82.2325 151.9555) (end 156.337 151.9555) (width 0.25) (layer B.Cu) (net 12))
 (segment (start 65.2145 150.1775) (end 80.4545 150.1775) (width 0.25) (layer B.Cu) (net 12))
 (segment (start 80.4545 150.1775) (end 82.2325 151.9555) (width 0.25) (layer B.Cu) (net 12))
 (segment (start 63.373 149.1615) (end 63.373 149.1615) (width 0.25) (layer F.Cu) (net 12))
 (segment (start 62.357 148.1455) (end 62.357 144.2085) (width 0.25) (layer F.Cu) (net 12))
 (segment (start 62.738 143.8275) (end 64.1985 143.8275) (width 0.25) (layer F.Cu) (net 12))
 (segment (start 62.357 144.2085) (end 62.738 143.8275) (width 0.25) (layer F.Cu) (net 12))
 (segment (start 80.518 148.2725) (end 80.4545 148.336) (width 0.25) (layer F.Cu) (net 12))
 (segment (start 83.451 148.2725) (end 80.518 148.2725) (width 0.25) (layer F.Cu) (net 12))
 (segment (start 80.4545 150.1775) (end 80.4545 148.336) (width 0.25) (layer B.Cu) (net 12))
 (segment (start 63.373 149.1615) (end 62.357 148.1455) (width 0.25) (layer F.Cu) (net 12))
 (via (at 63.373 149.1615) (size 0.8) (drill 0.4) (layers F.Cu B.Cu) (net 12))
 (segment (start 63.373 149.1615) (end 64.389 150.1775) (width 0.25) (layer B.Cu) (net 12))
 (segment (start 64.389 150.1775) (end 65.2145 150.1775) (width 0.25) (layer B.Cu) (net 12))
 (segment (start 162.437 148.2725) (end 162.437 146.2445) (width 0.25) (layer F.Cu) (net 30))
 (segment (start 162.437 146.2445) (end 161.544 145.3515) (width 0.25) (layer F.Cu) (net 30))
 (segment (start 161.544 145.3515) (end 156.1465 145.3515) (width 0.25) (layer F.Cu) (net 30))
 (segment (start 155.1345 146.3635) (end 155.1345 148.2725) (width 0.25) (layer F.Cu) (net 30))
 (segment (start 156.1465 145.3515) (end 155.1345 146.3635) (width 0.25) (layer F.Cu) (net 30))
 (segment (start 68.103499 145.002501) (end 69.2785 143.8275) (width 0.25) (layer F.Cu) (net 17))
 (segment (start 68.103499 149.065999) (end 68.103499 145.002501) (width 0.25) (layer F.Cu) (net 17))
 (segment (start 69.342 150.3045) (end 68.103499 149.065999) (width 0.25) (layer F.Cu) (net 17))
 (segment (start 110.9345 150.3045) (end 69.342 150.3045) (width 0.25) (layer F.Cu) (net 17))
 (segment (start 112.648 148.591) (end 110.9345 150.3045) (width 0.25) (layer F.Cu) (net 17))
 (segment (start 112.648 145.2245) (end 112.648 148.591) (width 0.25) (layer F.Cu) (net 17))
 (segment (start 122.7855 143.764) (end 121.2215 143.764) (width 0.25) (layer F.Cu) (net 18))
 (segment (start 121.2215 143.764) (end 120.0785 142.621) (width 0.25) (layer F.Cu) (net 18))
 (segment (start 120.0785 142.621) (end 113.03 142.621) (width 0.25) (layer F.Cu) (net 18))
 (segment (start 111.848 143.803) (end 111.848 145.2245) (width 0.25) (layer F.Cu) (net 18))
 (segment (start 113.03 142.621) (end 111.848 143.803) (width 0.25) (layer F.Cu) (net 18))
 (segment (start 73.183499 145.002501) (end 74.3585 143.8275) (width 0.25) (layer F.Cu) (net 18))
 (segment (start 73.183499 147.795999) (end 73.183499 145.002501) (width 0.25) (layer F.Cu) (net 18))
 (segment (start 74.4855 149.098) (end 73.183499 147.795999) (width 0.25) (layer F.Cu) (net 18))
 (segment (start 77.4065 149.098) (end 74.4855 149.098) (width 0.25) (layer F.Cu) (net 18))
 (segment (start 93.9165 146.1135) (end 80.391 146.1135) (width 0.25) (layer F.Cu) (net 18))
 (segment (start 97.409 149.606) (end 93.9165 146.1135) (width 0.25) (layer F.Cu) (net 18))
 (segment (start 110.4265 149.606) (end 97.409 149.606) (width 0.25) (layer F.Cu) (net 18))
 (segment (start 111.848 148.1845) (end 110.4265 149.606) (width 0.25) (layer F.Cu) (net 18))
 (segment (start 80.391 146.1135) (end 77.4065 149.098) (width 0.25) (layer F.Cu) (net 18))
 (segment (start 111.848 145.2245) (end 111.848 148.1845) (width 0.25) (layer F.Cu) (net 18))
 (segment (start 122.7855 141.7955) (end 112.776 141.7955) (width 0.25) (layer F.Cu) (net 19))
 (segment (start 111.048 143.5235) (end 111.048 145.2245) (width 0.25) (layer F.Cu) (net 19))
 (segment (start 112.776 141.7955) (end 111.048 143.5235) (width 0.25) (layer F.Cu) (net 19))
 (segment (start 74.3585 146.3675) (end 78.74 146.3675) (width 0.25) (layer F.Cu) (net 19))
 (segment (start 78.74 146.3675) (end 79.8195 145.288) (width 0.25) (layer F.Cu) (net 19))
 (segment (start 79.8195 145.288) (end 94.615 145.288) (width 0.25) (layer F.Cu) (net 19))
 (segment (start 94.615 145.288) (end 98.171 148.844) (width 0.25) (layer F.Cu) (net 19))
 (segment (start 98.171 148.844) (end 109.982 148.844) (width 0.25) (layer F.Cu) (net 19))
 (segment (start 111.048 147.778) (end 111.048 145.2245) (width 0.25) (layer F.Cu) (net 19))
 (segment (start 109.982 148.844) (end 111.048 147.778) (width 0.25) (layer F.Cu) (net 19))
 (segment (start 124.6105 141.7955) (end 124.6105 145.7325) (width 0.25) (layer F.Cu) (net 23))
 (via (at 70.612 140.589) (size 0.8) (drill 0.4) (layers F.Cu B.Cu) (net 23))
 (segment (start 70.643499 140.620499) (end 70.612 140.589) (width 0.25) (layer F.Cu) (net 23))
 (segment (start 70.643499 145.192499) (end 70.643499 140.620499) (width 0.25) (layer F.Cu) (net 23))
 (segment (start 71.8185 146.3675) (end 70.643499 145.192499) (width 0.25) (layer F.Cu) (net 23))
 (segment (start 70.612 140.589) (end 75.946 140.589) (width 0.25) (layer B.Cu) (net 23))
 (segment (start 81.4705 146.1135) (end 92.202 146.1135) (width 0.25) (layer B.Cu) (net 23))
 (segment (start 92.202 146.1135) (end 96.4565 150.368) (width 0.25) (layer B.Cu) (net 23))
 (segment (start 96.4565 150.368) (end 126.4285 150.368) (width 0.25) (layer B.Cu) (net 23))
 (via (at 127.9525 148.844) (size 0.8) (drill 0.4) (layers F.Cu B.Cu) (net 23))
 (segment (start 126.4285 150.368) (end 127.9525 148.844) (width 0.25) (layer B.Cu) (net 23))
 (segment (start 127.9525 148.844) (end 127.9525 147.1295) (width 0.25) (layer F.Cu) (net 23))
 (segment (start 126.5555 145.7325) (end 124.6105 145.7325) (width 0.25) (layer F.Cu) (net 23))
 (segment (start 127.9525 147.1295) (end 126.5555 145.7325) (width 0.25) (layer F.Cu) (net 23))
 (segment (start 124.6105 141.7955) (end 124.6105 140.6125) (width 0.25) (layer F.Cu) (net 23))
 (segment (start 124.6105 140.6125) (end 123.3805 139.3825) (width 0.25) (layer F.Cu) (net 23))
 (segment (start 123.3805 139.3825) (end 116.205 139.3825) (width 0.25) (layer F.Cu) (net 23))
 (segment (start 116.205 139.3825) (end 115.316 140.2715) (width 0.25) (layer F.Cu) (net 23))
 (segment (start 115.316 140.2715) (end 114.2365 140.2715) (width 0.25) (layer F.Cu) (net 23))
 (segment (start 114.2365 140.2715) (end 111.4425 140.2715) (width 0.25) (layer F.Cu) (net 23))
 (segment (start 111.4425 140.2715) (end 109.855 141.859) (width 0.25) (layer F.Cu) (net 23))
 (segment (start 109.855 141.859) (end 108.9025 141.859) (width 0.25) (layer F.Cu) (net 23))
 (via (at 108.204 141.1605) (size 0.8) (drill 0.4) (layers F.Cu B.Cu) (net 23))
 (segment (start 108.9025 141.859) (end 108.204 141.1605) (width 0.25) (layer F.Cu) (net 23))
 (via (at 108.204 138.1125) (size 0.8) (drill 0.4) (layers F.Cu B.Cu) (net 23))
 (segment (start 108.204 141.1605) (end 108.204 138.1125) (width 0.25) (layer B.Cu) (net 23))
 (segment (start 109.448 136.8685) (end 109.448 135.6945) (width 0.25) (layer F.Cu) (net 23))
 (segment (start 108.204 138.1125) (end 109.448 136.8685) (width 0.25) (layer F.Cu) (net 23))
 (segment (start 78.0415 146.1135) (end 77.0255 145.0975) (width 0.25) (layer B.Cu) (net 23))
 (segment (start 81.4705 146.1135) (end 78.0415 146.1135) (width 0.25) (layer B.Cu) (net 23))
 (segment (start 77.0255 141.6685) (end 75.946 140.589) (width 0.25) (layer B.Cu) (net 23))
 (segment (start 77.0255 145.0975) (end 77.0255 141.6685) (width 0.25) (layer B.Cu) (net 23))
 (segment (start 99.568 138.7475) (end 102.616 135.6995) (width 0.25) (layer F.Cu) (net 10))
 (segment (start 104.643 135.6995) (end 104.648 135.6945) (width 0.25) (layer F.Cu) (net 10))
 (segment (start 102.616 135.6995) (end 104.643 135.6995) (width 0.25) (layer F.Cu) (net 10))
 (segment (start 105.448 135.6945) (end 105.448 134.0865) (width 0.25) (layer F.Cu) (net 28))
 (segment (start 105.448 134.0865) (end 103.886 132.5245) (width 0.25) (layer F.Cu) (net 28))
 (segment (start 103.886 132.5245) (end 88.519 132.5245) (width 0.25) (layer F.Cu) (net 28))
 (segment (start 84.328 136.7155) (end 84.328 138.7475) (width 0.25) (layer F.Cu) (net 28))
 (segment (start 88.519 132.5245) (end 84.328 136.7155) (width 0.25) (layer F.Cu) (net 28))
 (segment (start 106.248 135.6945) (end 106.248 133.172) (width 0.25) (layer F.Cu) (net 13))
 (segment (start 104.394 131.318) (end 69.1515 131.318) (width 0.25) (layer F.Cu) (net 13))
 (segment (start 106.248 133.172) (end 104.394 131.318) (width 0.25) (layer F.Cu) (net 13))
 (segment (start 84.328 123.7615) (end 90.17 123.7615) (width 0.25) (layer F.Cu) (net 9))
 (segment (start 90.17 123.7615) (end 94.742 128.3335) (width 0.25) (layer F.Cu) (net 9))
 (segment (start 94.742 128.3335) (end 103.8225 128.3335) (width 0.25) (layer F.Cu) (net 9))
 (segment (start 107.048 131.559) (end 107.048 135.6945) (width 0.25) (layer F.Cu) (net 9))
 (segment (start 103.8225 128.3335) (end 107.048 131.559) (width 0.25) (layer F.Cu) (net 9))
 (segment (start 107.848 135.6945) (end 107.848 130.3905) (width 0.25) (layer F.Cu) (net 8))
 (segment (start 101.219 123.7615) (end 99.568 123.7615) (width 0.25) (layer F.Cu) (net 8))
 (segment (start 107.848 130.3905) (end 101.219 123.7615) (width 0.25) (layer F.Cu) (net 8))
 (segment (start 108.648 135.6945) (end 108.648 124.397) (width 0.25) (layer F.Cu) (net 6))
 (segment (start 109.2835 123.7615) (end 114.808 123.7615) (width 0.25) (layer F.Cu) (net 6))
 (segment (start 108.648 124.397) (end 109.2835 123.7615) (width 0.25) (layer F.Cu) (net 6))
 (segment (start 111.848 127.3565) (end 111.848 135.6945) (width 0.25) (layer F.Cu) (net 4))
 (segment (start 112.903 126.3015) (end 111.848 127.3565) (width 0.25) (layer F.Cu) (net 4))
 (segment (start 127.6985 126.3015) (end 112.903 126.3015) (width 0.25) (layer F.Cu) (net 4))
 (segment (start 130.2385 123.7615) (end 127.6985 126.3015) (width 0.25) (layer F.Cu) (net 4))
 (segment (start 112.648 135.6945) (end 112.648 128.4615) (width 0.25) (layer F.Cu) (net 2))
 (segment (start 140.7785 128.4615) (end 145.4785 123.7615) (width 0.25) (layer F.Cu) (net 2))
 (segment (start 112.648 128.4615) (end 140.7785 128.4615) (width 0.25) (layer F.Cu) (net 2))
 (segment (start 113.448 135.6945) (end 113.448 132.2335) (width 0.25) (layer F.Cu) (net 1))
 (segment (start 114.3635 131.318) (end 160.528 131.318) (width 0.25) (layer F.Cu) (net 1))
 (segment (start 113.448 132.2335) (end 114.3635 131.318) (width 0.25) (layer F.Cu) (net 1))
 (segment (start 145.4475 138.757) (end 145.4475 133.3825) (width 0.25) (layer F.Cu) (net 3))
 (segment (start 145.4475 133.3825) (end 144.2085 132.1435) (width 0.25) (layer F.Cu) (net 3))
 (segment (start 144.2085 132.1435) (end 115.57 132.1435) (width 0.25) (layer F.Cu) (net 3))
 (segment (start 114.248 133.4655) (end 114.248 135.6945) (width 0.25) (layer F.Cu) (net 3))
 (segment (start 115.57 132.1435) (end 114.248 133.4655) (width 0.25) (layer F.Cu) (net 3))
 (segment (start 115.048 135.6945) (end 115.048 133.8085) (width 0.25) (layer F.Cu) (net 5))
 (segment (start 115.048 133.8085) (end 115.697 133.1595) (width 0.25) (layer F.Cu) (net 5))
 (segment (start 124.6505 133.1595) (end 130.2385 138.7475) (width 0.25) (layer F.Cu) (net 5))
 (segment (start 115.697 133.1595) (end 124.6505 133.1595) (width 0.25) (layer F.Cu) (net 5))
 (segment (start 115.848 137.7075) (end 115.848 135.6945) (width 0.25) (layer F.Cu) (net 7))
 (segment (start 114.808 138.7475) (end 115.848 137.7075) (width 0.25) (layer F.Cu) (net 7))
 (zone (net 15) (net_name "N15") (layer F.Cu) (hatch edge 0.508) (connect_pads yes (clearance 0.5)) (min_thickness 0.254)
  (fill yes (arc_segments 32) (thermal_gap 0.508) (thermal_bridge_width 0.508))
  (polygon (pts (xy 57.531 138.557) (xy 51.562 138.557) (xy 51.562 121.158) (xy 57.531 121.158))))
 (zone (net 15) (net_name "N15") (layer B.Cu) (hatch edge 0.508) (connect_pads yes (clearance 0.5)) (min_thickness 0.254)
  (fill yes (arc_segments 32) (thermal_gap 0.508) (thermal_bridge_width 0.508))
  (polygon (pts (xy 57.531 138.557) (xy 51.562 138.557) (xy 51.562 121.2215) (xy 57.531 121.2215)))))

